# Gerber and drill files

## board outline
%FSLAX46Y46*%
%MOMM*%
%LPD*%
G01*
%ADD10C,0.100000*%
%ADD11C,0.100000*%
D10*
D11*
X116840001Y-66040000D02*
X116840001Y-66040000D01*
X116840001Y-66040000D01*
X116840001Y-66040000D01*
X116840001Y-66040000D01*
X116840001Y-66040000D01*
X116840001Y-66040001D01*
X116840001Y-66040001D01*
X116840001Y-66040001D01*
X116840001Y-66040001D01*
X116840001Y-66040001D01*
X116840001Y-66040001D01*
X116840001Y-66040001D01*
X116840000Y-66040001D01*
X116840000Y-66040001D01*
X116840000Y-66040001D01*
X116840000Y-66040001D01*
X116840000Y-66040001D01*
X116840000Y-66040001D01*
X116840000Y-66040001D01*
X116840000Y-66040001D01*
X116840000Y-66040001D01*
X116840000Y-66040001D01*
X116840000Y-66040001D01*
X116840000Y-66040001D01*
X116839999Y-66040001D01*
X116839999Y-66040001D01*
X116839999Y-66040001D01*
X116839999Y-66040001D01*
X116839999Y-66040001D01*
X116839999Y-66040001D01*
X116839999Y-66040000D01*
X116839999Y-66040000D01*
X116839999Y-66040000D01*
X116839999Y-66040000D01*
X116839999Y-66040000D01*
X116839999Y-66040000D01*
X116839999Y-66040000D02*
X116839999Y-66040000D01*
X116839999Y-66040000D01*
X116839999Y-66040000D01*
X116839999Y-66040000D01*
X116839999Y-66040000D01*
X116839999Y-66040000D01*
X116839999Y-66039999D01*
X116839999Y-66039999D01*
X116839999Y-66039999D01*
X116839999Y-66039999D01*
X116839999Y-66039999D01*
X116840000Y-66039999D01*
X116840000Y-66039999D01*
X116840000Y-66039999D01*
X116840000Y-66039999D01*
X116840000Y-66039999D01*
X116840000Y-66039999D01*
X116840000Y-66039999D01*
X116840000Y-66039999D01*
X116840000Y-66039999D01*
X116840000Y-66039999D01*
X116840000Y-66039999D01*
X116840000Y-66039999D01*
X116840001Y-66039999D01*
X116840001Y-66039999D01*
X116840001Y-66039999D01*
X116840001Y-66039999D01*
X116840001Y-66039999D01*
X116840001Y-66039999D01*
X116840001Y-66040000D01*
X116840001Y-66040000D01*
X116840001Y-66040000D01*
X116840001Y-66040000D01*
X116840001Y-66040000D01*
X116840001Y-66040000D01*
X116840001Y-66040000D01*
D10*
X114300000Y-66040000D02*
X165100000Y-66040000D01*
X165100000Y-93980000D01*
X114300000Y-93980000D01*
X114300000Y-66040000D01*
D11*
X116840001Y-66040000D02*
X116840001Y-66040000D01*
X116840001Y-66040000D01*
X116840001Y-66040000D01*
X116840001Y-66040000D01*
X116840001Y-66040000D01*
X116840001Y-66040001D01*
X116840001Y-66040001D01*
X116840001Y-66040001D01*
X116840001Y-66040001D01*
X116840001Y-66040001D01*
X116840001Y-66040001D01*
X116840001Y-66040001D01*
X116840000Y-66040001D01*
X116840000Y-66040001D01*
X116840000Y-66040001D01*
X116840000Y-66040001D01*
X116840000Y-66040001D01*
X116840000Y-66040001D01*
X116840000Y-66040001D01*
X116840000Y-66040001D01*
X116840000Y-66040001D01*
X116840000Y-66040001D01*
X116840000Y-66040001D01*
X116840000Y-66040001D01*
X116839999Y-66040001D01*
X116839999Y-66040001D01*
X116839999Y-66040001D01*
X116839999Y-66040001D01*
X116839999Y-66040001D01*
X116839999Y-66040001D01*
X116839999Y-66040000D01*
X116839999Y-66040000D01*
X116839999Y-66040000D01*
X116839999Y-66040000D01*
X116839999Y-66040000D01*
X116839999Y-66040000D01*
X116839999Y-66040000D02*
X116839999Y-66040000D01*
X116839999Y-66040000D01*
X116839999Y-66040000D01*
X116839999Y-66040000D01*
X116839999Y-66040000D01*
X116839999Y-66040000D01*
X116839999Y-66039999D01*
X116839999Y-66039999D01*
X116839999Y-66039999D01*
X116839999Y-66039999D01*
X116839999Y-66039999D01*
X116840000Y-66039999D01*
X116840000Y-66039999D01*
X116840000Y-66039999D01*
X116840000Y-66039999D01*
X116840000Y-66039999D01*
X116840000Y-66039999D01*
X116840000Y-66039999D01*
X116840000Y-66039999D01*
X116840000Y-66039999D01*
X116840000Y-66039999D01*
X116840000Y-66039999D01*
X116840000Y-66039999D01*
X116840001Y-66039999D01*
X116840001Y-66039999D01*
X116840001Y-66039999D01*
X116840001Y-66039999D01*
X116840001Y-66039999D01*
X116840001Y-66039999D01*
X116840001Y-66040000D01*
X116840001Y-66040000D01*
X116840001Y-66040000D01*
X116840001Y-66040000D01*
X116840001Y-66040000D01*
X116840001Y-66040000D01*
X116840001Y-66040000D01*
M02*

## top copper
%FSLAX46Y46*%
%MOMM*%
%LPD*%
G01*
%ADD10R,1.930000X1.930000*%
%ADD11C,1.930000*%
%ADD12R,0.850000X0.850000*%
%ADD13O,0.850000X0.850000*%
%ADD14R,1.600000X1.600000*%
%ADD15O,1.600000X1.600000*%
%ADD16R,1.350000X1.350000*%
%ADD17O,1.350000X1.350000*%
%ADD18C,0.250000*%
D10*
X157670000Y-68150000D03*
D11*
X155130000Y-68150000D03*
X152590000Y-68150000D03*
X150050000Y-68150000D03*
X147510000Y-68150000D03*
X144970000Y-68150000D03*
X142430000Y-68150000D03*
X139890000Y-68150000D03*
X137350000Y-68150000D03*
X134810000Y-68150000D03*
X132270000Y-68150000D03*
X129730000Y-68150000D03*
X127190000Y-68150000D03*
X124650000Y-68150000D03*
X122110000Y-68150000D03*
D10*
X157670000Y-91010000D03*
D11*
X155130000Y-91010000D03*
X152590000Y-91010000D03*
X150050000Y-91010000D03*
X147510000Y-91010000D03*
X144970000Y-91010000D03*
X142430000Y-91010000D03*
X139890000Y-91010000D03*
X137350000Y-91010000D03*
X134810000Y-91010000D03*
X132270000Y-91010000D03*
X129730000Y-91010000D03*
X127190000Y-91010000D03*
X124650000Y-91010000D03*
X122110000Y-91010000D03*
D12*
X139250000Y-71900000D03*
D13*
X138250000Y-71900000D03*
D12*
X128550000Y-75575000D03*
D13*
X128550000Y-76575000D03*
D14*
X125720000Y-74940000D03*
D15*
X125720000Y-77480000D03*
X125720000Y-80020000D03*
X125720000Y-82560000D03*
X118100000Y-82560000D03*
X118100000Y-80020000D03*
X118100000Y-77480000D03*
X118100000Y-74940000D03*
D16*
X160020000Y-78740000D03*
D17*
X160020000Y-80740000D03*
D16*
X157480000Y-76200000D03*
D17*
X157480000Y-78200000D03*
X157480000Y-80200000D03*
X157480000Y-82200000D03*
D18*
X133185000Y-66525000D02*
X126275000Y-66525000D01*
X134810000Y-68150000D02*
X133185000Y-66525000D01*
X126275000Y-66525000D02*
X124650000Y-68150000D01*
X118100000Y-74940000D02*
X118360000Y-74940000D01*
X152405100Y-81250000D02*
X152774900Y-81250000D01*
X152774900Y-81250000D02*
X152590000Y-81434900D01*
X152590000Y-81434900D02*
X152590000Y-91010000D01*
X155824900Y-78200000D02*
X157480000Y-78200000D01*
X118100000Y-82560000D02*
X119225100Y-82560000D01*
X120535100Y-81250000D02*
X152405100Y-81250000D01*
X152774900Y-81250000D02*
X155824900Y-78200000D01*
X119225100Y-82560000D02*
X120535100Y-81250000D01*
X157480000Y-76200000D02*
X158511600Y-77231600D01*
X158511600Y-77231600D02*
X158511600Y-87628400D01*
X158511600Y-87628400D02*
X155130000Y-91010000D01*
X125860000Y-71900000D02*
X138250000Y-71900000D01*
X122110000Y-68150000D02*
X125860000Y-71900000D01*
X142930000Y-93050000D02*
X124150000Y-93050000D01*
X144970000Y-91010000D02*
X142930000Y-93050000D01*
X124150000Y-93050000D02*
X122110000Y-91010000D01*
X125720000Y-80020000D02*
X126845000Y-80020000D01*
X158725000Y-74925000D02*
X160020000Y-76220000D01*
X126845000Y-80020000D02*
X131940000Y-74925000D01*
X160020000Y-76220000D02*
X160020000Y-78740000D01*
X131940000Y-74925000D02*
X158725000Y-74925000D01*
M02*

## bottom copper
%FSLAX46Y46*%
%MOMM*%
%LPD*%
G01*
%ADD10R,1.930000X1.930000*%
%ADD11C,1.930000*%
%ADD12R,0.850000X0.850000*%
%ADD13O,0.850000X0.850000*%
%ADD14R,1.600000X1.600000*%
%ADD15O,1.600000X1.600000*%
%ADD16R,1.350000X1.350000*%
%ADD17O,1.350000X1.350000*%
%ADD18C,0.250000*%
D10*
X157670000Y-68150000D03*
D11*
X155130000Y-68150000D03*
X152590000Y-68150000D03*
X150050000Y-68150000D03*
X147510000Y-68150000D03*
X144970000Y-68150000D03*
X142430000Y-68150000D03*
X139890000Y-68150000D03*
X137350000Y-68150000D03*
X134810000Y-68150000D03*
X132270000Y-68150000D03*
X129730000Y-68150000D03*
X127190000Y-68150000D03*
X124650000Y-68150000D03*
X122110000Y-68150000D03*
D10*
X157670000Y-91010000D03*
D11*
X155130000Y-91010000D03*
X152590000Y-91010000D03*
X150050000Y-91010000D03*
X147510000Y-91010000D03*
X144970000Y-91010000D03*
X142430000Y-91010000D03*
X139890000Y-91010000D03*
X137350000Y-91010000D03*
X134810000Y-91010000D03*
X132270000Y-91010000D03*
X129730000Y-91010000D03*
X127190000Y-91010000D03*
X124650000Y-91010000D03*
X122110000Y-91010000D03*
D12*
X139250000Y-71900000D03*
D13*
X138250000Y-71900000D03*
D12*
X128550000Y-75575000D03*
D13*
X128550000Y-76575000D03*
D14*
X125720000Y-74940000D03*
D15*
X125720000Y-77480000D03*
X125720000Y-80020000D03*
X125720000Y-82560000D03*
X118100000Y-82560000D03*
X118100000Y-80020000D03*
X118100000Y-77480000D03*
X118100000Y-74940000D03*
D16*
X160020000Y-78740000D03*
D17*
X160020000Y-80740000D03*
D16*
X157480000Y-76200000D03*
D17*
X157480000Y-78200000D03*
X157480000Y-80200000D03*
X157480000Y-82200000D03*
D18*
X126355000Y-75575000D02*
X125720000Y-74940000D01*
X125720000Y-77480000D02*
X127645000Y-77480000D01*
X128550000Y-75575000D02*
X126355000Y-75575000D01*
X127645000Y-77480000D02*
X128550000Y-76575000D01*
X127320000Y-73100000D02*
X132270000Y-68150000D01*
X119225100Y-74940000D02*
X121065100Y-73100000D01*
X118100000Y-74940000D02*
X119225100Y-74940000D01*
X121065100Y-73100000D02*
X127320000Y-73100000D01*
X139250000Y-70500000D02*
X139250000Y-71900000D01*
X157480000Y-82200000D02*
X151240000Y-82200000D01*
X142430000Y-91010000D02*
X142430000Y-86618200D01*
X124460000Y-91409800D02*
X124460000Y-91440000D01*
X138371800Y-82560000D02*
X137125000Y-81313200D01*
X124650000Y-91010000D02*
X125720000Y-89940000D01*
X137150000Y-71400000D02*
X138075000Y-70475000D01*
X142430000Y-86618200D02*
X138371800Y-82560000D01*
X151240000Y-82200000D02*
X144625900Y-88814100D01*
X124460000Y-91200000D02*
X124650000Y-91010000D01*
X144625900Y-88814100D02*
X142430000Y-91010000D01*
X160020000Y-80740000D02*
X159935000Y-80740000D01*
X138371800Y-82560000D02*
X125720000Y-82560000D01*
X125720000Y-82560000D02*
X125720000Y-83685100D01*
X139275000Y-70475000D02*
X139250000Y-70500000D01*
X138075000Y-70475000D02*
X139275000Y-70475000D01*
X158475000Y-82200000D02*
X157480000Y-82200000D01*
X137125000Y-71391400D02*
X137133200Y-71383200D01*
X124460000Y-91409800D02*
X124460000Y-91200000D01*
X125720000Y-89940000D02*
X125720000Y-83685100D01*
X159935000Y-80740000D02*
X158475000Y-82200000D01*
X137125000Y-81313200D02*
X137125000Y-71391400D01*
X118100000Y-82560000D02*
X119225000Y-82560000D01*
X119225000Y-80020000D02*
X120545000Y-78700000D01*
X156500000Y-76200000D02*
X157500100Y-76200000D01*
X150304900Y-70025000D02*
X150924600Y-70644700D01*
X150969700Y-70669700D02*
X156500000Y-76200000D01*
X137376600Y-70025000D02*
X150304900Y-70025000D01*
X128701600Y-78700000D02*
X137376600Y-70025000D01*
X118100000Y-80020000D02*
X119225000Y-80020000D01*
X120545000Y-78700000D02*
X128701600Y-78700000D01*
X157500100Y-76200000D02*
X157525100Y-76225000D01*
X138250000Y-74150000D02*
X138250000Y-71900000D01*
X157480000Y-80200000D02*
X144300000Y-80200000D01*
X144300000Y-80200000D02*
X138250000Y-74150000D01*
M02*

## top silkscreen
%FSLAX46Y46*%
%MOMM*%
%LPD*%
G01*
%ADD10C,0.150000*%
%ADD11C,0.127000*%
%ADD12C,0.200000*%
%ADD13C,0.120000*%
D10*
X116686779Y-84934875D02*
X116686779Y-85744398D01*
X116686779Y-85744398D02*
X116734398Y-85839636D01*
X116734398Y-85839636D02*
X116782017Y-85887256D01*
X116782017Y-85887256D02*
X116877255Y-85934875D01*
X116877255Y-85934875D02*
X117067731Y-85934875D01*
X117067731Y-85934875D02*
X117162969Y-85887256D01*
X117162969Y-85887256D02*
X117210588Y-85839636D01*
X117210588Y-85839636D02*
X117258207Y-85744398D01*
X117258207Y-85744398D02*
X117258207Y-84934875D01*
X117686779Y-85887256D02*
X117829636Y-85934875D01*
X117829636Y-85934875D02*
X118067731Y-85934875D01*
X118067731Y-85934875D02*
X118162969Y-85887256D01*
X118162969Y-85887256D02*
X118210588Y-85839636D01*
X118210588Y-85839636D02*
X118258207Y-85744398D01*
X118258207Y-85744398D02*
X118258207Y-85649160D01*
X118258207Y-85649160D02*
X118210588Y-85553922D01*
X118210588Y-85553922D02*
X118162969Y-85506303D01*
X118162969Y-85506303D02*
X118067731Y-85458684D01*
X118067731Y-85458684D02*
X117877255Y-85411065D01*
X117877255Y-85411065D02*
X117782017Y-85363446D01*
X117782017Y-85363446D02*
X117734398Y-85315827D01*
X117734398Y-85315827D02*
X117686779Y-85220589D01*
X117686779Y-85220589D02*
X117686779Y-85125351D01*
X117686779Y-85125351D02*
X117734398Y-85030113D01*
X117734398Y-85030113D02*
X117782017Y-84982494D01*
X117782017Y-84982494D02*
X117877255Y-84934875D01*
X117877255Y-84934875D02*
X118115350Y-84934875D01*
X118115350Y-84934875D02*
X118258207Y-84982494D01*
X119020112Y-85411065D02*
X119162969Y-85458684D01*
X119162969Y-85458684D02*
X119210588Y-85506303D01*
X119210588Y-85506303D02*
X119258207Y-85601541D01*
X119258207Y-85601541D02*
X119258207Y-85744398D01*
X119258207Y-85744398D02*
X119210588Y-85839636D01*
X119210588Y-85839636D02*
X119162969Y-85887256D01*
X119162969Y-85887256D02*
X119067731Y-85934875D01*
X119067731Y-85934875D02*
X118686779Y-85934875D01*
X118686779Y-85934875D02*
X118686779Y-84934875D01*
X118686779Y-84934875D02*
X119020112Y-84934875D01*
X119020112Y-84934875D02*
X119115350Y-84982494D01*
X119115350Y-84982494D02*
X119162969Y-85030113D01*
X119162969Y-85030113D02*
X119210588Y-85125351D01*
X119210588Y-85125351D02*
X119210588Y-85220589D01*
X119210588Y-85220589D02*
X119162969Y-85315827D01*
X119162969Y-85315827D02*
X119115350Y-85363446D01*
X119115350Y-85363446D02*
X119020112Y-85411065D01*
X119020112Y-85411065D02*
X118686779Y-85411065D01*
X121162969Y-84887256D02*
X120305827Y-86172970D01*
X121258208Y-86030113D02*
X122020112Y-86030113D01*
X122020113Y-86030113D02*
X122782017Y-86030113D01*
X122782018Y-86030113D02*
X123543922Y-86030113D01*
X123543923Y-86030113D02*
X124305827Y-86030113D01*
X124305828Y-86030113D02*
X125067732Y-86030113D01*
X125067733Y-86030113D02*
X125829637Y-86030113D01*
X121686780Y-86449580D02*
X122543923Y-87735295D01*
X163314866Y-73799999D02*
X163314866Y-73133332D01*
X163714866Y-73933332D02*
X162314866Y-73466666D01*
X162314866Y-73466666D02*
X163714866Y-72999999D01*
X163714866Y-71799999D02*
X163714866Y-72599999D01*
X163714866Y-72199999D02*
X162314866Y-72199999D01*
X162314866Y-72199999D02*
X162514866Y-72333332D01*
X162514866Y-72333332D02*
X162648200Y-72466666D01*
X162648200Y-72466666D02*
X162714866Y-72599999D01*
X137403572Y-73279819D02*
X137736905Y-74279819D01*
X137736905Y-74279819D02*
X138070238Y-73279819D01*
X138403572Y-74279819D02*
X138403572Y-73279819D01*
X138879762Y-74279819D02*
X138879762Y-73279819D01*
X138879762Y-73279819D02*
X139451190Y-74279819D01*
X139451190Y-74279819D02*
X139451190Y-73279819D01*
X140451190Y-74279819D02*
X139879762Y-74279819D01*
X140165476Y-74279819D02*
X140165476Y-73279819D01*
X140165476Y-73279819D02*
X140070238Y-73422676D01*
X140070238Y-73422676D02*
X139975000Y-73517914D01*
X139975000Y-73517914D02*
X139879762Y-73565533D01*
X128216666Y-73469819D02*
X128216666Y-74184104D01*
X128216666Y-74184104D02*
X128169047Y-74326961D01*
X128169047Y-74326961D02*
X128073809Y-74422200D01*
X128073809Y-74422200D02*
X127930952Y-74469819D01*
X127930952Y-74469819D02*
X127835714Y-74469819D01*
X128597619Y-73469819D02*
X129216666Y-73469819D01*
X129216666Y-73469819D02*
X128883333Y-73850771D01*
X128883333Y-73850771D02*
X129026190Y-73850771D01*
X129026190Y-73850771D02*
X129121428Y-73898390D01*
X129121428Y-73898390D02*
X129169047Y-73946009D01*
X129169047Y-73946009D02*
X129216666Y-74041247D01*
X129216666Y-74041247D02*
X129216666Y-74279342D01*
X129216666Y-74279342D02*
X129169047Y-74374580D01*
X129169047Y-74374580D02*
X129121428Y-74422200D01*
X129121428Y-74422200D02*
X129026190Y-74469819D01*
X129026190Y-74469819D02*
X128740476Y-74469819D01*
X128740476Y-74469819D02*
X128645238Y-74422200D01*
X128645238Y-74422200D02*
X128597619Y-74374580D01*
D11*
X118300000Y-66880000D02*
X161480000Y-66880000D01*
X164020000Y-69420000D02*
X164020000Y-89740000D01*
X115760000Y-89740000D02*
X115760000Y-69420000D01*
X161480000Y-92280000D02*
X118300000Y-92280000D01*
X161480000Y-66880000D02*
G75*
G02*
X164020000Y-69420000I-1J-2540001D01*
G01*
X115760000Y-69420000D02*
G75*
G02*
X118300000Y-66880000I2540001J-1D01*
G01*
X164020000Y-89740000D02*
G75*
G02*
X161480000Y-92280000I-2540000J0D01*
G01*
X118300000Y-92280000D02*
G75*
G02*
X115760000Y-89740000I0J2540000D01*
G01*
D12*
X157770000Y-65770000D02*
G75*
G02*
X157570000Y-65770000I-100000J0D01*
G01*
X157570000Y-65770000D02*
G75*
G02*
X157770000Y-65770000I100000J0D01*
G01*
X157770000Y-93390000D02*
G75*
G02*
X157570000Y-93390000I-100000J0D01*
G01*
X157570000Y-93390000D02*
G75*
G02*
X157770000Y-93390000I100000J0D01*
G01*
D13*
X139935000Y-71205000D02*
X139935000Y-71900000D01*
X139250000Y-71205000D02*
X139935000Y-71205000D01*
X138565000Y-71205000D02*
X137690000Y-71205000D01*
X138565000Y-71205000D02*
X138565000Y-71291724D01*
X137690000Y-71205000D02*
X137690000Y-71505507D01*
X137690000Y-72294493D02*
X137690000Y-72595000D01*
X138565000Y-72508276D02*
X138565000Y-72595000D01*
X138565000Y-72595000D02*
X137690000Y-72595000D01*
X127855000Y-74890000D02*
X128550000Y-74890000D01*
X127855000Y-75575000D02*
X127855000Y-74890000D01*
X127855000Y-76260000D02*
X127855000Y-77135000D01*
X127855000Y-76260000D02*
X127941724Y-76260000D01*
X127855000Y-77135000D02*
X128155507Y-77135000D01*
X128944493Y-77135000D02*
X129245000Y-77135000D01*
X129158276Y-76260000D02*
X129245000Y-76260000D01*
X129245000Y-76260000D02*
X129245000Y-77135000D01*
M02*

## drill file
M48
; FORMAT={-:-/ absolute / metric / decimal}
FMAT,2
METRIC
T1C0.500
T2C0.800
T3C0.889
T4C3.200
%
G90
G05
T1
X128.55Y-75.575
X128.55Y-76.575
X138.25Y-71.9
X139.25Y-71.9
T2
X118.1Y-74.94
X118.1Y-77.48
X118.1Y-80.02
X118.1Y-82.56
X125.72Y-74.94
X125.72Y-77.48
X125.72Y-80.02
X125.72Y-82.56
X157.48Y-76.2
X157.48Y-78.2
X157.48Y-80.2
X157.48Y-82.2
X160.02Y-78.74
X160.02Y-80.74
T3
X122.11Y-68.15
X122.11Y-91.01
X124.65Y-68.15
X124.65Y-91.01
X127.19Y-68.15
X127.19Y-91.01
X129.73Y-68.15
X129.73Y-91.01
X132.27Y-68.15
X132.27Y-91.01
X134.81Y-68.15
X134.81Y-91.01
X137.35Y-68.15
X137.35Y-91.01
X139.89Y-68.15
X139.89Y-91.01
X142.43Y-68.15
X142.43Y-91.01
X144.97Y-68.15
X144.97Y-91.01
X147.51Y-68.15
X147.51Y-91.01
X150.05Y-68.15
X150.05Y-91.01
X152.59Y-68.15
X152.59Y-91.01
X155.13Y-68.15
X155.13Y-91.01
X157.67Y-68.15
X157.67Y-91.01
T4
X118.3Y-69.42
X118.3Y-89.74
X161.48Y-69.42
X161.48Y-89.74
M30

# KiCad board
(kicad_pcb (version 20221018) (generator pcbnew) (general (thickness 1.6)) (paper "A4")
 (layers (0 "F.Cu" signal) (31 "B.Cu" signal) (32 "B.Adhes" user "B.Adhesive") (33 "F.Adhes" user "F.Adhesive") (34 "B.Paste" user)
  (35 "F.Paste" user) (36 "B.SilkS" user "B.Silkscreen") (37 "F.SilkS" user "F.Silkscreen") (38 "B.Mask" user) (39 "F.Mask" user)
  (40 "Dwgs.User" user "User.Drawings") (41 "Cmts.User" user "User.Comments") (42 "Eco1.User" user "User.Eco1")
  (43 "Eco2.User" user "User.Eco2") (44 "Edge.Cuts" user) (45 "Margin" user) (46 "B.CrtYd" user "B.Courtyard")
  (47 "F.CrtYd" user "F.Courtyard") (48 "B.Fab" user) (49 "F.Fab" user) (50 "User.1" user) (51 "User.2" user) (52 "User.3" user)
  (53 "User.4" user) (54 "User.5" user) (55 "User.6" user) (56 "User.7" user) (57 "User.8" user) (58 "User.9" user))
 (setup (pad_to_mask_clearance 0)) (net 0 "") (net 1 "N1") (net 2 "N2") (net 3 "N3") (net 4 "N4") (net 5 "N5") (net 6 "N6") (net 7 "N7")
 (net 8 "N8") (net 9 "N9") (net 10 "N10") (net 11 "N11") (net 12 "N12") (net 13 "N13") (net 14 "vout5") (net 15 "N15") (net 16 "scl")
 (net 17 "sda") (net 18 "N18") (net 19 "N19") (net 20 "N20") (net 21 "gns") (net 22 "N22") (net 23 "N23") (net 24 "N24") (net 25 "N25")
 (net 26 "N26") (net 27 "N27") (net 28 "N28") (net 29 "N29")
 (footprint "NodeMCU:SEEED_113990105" (layer "F.Cu") (at 139.89 79.58 -90)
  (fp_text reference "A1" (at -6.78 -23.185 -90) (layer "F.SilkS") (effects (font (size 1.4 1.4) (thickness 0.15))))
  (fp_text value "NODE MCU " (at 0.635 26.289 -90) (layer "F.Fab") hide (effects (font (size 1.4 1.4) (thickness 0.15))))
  (fp_line (start -12.7 21.59) (end -12.7 -21.59) (stroke (width 0.127) (type solid)) (layer "F.SilkS"))
  (fp_line (start -10.16 -24.13) (end 10.16 -24.13) (stroke (width 0.127) (type solid)) (layer "F.SilkS"))
  (fp_line (start 10.16 24.13) (end -10.16 24.13) (stroke (width 0.127) (type solid)) (layer "F.SilkS"))
  (fp_line (start 12.7 -21.59) (end 12.7 21.59) (stroke (width 0.127) (type solid)) (layer "F.SilkS"))
  (fp_arc (start -12.7 -21.59) (mid -11.956051 -23.386051) (end -10.16 -24.13) (stroke (width 0.127) (type solid)) (layer "F.SilkS"))
  (fp_arc (start -10.16 24.13) (mid -11.956051 23.386051) (end -12.7 21.59) (stroke (width 0.127) (type solid)) (layer "F.SilkS"))
  (fp_arc (start 10.16 -24.13) (mid 11.956051 -23.386051) (end 12.7 -21.59) (stroke (width 0.127) (type solid)) (layer "F.SilkS"))
  (fp_arc (start 12.7 21.59) (mid 11.956051 23.386051) (end 10.16 24.13) (stroke (width 0.127) (type solid)) (layer "F.SilkS"))
  (fp_circle (center -13.81 -17.78) (end -13.71 -17.78) (stroke (width 0.2) (type solid)) (fill none) (layer "F.SilkS"))
  (fp_circle (center 13.81 -17.78) (end 13.91 -17.78) (stroke (width 0.2) (type solid)) (fill none) (layer "F.SilkS"))
  (pad "" np_thru_hole circle (at -10.16 -21.59 270) (size 3.2 3.2) (drill 3.2) (layers "*.Cu" "*.Mask"))
  (pad "" np_thru_hole circle (at -10.16 21.59 270) (size 3.2 3.2) (drill 3.2) (layers "*.Cu" "*.Mask"))
  (pad "" np_thru_hole circle (at 10.16 -21.59 270) (size 3.2 3.2) (drill 3.2) (layers "*.Cu" "*.Mask"))
  (pad "" np_thru_hole circle (at 10.16 21.59 270) (size 3.2 3.2) (drill 3.2) (layers "*.Cu" "*.Mask"))
  (pad "J1_1" thru_hole rect (at -11.43 -17.78 270) (size 1.93 1.93) (drill 0.889) (layers "*.Cu" "*.Mask") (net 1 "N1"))
  (pad "J1_2" thru_hole circle (at -11.43 -15.24 270) (size 1.93 1.93) (drill 0.889) (layers "*.Cu" "*.Mask") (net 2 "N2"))
  (pad "J1_3" thru_hole circle (at -11.43 -12.7 270) (size 1.93 1.93) (drill 0.889) (layers "*.Cu" "*.Mask") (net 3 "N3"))
  (pad "J1_4" thru_hole circle (at -11.43 -10.16 270) (size 1.93 1.93) (drill 0.889) (layers "*.Cu" "*.Mask") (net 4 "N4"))
  (pad "J1_5" thru_hole circle (at -11.43 -7.62 270) (size 1.93 1.93) (drill 0.889) (layers "*.Cu" "*.Mask") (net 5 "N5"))
  (pad "J1_6" thru_hole circle (at -11.43 -5.08 270) (size 1.93 1.93) (drill 0.889) (layers "*.Cu" "*.Mask") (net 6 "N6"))
  (pad "J1_7" thru_hole circle (at -11.43 -2.54 270) (size 1.93 1.93) (drill 0.889) (layers "*.Cu" "*.Mask") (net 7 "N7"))
  (pad "J1_8" thru_hole circle (at -11.43 0 270) (size 1.93 1.93) (drill 0.889) (layers "*.Cu" "*.Mask") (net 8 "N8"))
  (pad "J1_9" thru_hole circle (at -11.43 2.54 270) (size 1.93 1.93) (drill 0.889) (layers "*.Cu" "*.Mask") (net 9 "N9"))
  (pad "J1_10" thru_hole circle (at -11.43 5.08 270) (size 1.93 1.93) (drill 0.889) (layers "*.Cu" "*.Mask") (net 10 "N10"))
  (pad "J1_11" thru_hole circle (at -11.43 7.62 270) (size 1.93 1.93) (drill 0.889) (layers "*.Cu" "*.Mask") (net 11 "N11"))
  (pad "J1_12" thru_hole circle (at -11.43 10.16 270) (size 1.93 1.93) (drill 0.889) (layers "*.Cu" "*.Mask") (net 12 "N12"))
  (pad "J1_13" thru_hole circle (at -11.43 12.7 270) (size 1.93 1.93) (drill 0.889) (layers "*.Cu" "*.Mask") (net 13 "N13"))
  (pad "J1_14" thru_hole circle (at -11.43 15.24 270) (size 1.93 1.93) (drill 0.889) (layers "*.Cu" "*.Mask") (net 10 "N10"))
  (pad "J1_15" thru_hole circle (at -11.43 17.78 270) (size 1.93 1.93) (drill 0.889) (layers "*.Cu" "*.Mask") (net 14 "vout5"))
  (pad "J2_1" thru_hole rect (at 11.43 -17.78 270) (size 1.93 1.93) (drill 0.889) (layers "*.Cu" "*.Mask") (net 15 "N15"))
  (pad "J2_2" thru_hole circle (at 11.43 -15.24 270) (size 1.93 1.93) (drill 0.889) (layers "*.Cu" "*.Mask") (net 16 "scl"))
  (pad "J2_3" thru_hole circle (at 11.43 -12.7 270) (size 1.93 1.93) (drill 0.889) (layers "*.Cu" "*.Mask") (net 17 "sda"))
  (pad "J2_4" thru_hole circle (at 11.43 -10.16 270) (size 1.93 1.93) (drill 0.889) (layers "*.Cu" "*.Mask") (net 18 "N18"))
  (pad "J2_5" thru_hole circle (at 11.43 -7.62 270) (size 1.93 1.93) (drill 0.889) (layers "*.Cu" "*.Mask") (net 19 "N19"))
  (pad "J2_6" thru_hole circle (at 11.43 -5.08 270) (size 1.93 1.93) (drill 0.889) (layers "*.Cu" "*.Mask") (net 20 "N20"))
  (pad "J2_7" thru_hole circle (at 11.43 -2.54 270) (size 1.93 1.93) (drill 0.889) (layers "*.Cu" "*.Mask") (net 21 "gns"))
  (pad "J2_8" thru_hole circle (at 11.43 0 270) (size 1.93 1.93) (drill 0.889) (layers "*.Cu" "*.Mask") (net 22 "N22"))
  (pad "J2_9" thru_hole circle (at 11.43 2.54 270) (size 1.93 1.93) (drill 0.889) (layers "*.Cu" "*.Mask") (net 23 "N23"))
  (pad "J2_10" thru_hole circle (at 11.43 5.08 270) (size 1.93 1.93) (drill 0.889) (layers "*.Cu" "*.Mask") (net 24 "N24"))
  (pad "J2_11" thru_hole circle (at 11.43 7.62 270) (size 1.93 1.93) (drill 0.889) (layers "*.Cu" "*.Mask") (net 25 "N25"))
  (pad "J2_12" thru_hole circle (at 11.43 10.16 270) (size 1.93 1.93) (drill 0.889) (layers "*.Cu" "*.Mask") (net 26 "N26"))
  (pad "J2_13" thru_hole circle (at 11.43 12.7 270) (size 1.93 1.93) (drill 0.889) (layers "*.Cu" "*.Mask") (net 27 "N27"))
  (pad "J2_14" thru_hole circle (at 11.43 15.24 270) (size 1.93 1.93) (drill 0.889) (layers "*.Cu" "*.Mask") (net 21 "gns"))
  (pad "J2_15" thru_hole circle (at 11.43 17.78 270) (size 1.93 1.93) (drill 0.889) (layers "*.Cu" "*.Mask") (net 20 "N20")))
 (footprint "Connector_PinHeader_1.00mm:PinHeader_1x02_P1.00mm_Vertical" (layer "F.Cu") (at 139.25 71.9 -90)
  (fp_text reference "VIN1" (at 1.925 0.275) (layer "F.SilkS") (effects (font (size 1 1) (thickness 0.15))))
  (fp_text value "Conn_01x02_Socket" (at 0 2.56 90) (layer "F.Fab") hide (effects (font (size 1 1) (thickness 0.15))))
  (fp_line (start -0.695 -0.685) (end 0 -0.685) (stroke (width 0.12) (type solid)) (layer "F.SilkS"))
  (fp_line (start -0.695 0) (end -0.695 -0.685) (stroke (width 0.12) (type solid)) (layer "F.SilkS"))
  (fp_line (start -0.695 0.685) (end -0.695 1.56) (stroke (width 0.12) (type solid)) (layer "F.SilkS"))
  (fp_line (start -0.695 0.685) (end -0.608276 0.685) (stroke (width 0.12) (type solid)) (layer "F.SilkS"))
  (fp_line (start -0.695 1.56) (end -0.394493 1.56) (stroke (width 0.12) (type solid)) (layer "F.SilkS"))
  (fp_line (start 0.394493 1.56) (end 0.695 1.56) (stroke (width 0.12) (type solid)) (layer "F.SilkS"))
  (fp_line (start 0.608276 0.685) (end 0.695 0.685) (stroke (width 0.12) (type solid)) (layer "F.SilkS"))
  (fp_line (start 0.695 0.685) (end 0.695 1.56) (stroke (width 0.12) (type solid)) (layer "F.SilkS"))
  (pad "1" thru_hole rect (at 0 0 270) (size 0.85 0.85) (drill 0.5) (layers "*.Cu" "*.Mask") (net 21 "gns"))
  (pad "2" thru_hole oval (at 0 1 270) (size 0.85 0.85) (drill 0.5) (layers "*.Cu" "*.Mask") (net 14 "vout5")))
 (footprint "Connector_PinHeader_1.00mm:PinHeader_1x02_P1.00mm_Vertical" (layer "F.Cu") (at 128.55 75.575)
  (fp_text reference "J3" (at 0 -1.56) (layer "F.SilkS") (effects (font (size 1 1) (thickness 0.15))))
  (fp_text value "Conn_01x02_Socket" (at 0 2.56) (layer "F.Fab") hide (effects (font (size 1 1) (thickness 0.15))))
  (fp_line (start -0.695 -0.685) (end 0 -0.685) (stroke (width 0.12) (type solid)) (layer "F.SilkS"))
  (fp_line (start -0.695 0) (end -0.695 -0.685) (stroke (width 0.12) (type solid)) (layer "F.SilkS"))
  (fp_line (start -0.695 0.685) (end -0.695 1.56) (stroke (width 0.12) (type solid)) (layer "F.SilkS"))
  (fp_line (start -0.695 0.685) (end -0.608276 0.685) (stroke (width 0.12) (type solid)) (layer "F.SilkS"))
  (fp_line (start -0.695 1.56) (end -0.394493 1.56) (stroke (width 0.12) (type solid)) (layer "F.SilkS"))
  (fp_line (start 0.394493 1.56) (end 0.695 1.56) (stroke (width 0.12) (type solid)) (layer "F.SilkS"))
  (fp_line (start 0.608276 0.685) (end 0.695 0.685) (stroke (width 0.12) (type solid)) (layer "F.SilkS"))
  (fp_line (start 0.695 0.685) (end 0.695 1.56) (stroke (width 0.12) (type solid)) (layer "F.SilkS"))
  (pad "1" thru_hole rect (at 0 0) (size 0.85 0.85) (drill 0.5) (layers "*.Cu" "*.Mask"))
  (pad "2" thru_hole oval (at 0 1) (size 0.85 0.85) (drill 0.5) (layers "*.Cu" "*.Mask")))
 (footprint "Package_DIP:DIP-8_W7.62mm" (layer "B.Cu") (at 125.72 74.94 180)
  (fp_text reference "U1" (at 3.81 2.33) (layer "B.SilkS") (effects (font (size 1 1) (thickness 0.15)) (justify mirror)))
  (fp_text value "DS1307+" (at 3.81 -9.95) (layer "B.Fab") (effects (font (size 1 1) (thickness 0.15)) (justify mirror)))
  (pad "1" thru_hole rect (at 0 0 180) (size 1.6 1.6) (drill 0.8) (layers "*.Cu" "*.Mask"))
  (pad "2" thru_hole oval (at 0 -2.54 180) (size 1.6 1.6) (drill 0.8) (layers "*.Cu" "*.Mask"))
  (pad "3" thru_hole oval (at 0 -5.08 180) (size 1.6 1.6) (drill 0.8) (layers "*.Cu" "*.Mask") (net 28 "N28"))
  (pad "4" thru_hole oval (at 0 -7.62 180) (size 1.6 1.6) (drill 0.8) (layers "*.Cu" "*.Mask") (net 21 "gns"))
  (pad "5" thru_hole oval (at 7.62 -7.62 180) (size 1.6 1.6) (drill 0.8) (layers "*.Cu" "*.Mask") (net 17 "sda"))
  (pad "6" thru_hole oval (at 7.62 -5.08 180) (size 1.6 1.6) (drill 0.8) (layers "*.Cu" "*.Mask") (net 16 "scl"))
  (pad "7" thru_hole oval (at 7.62 -2.54 180) (size 1.6 1.6) (drill 0.8) (layers "*.Cu" "*.Mask") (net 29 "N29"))
  (pad "8" thru_hole oval (at 7.62 0 180) (size 1.6 1.6) (drill 0.8) (layers "*.Cu" "*.Mask") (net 11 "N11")))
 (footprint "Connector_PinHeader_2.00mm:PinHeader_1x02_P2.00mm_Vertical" (layer "B.Cu") (at 160.02 78.74 180)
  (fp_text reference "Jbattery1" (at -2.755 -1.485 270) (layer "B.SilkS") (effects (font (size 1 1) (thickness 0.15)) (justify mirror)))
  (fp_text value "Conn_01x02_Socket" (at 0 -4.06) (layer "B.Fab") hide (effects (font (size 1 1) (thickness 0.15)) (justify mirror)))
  (pad "1" thru_hole rect (at 0 0 180) (size 1.35 1.35) (drill 0.8) (layers "*.Cu" "*.Mask") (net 28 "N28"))
  (pad "2" thru_hole oval (at 0 -2 180) (size 1.35 1.35) (drill 0.8) (layers "*.Cu" "*.Mask") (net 21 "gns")))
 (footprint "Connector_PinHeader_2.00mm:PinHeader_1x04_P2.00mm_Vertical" (layer "B.Cu") (at 157.48 76.2 180)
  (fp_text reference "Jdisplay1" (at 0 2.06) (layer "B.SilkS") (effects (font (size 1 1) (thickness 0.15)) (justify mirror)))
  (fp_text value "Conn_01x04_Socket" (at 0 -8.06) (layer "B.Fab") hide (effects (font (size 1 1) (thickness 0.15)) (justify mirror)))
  (pad "1" thru_hole rect (at 0 0 180) (size 1.35 1.35) (drill 0.8) (layers "*.Cu" "*.Mask") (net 16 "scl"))
  (pad "2" thru_hole oval (at 0 -2 180) (size 1.35 1.35) (drill 0.8) (layers "*.Cu" "*.Mask") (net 17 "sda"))
  (pad "3" thru_hole oval (at 0 -4 180) (size 1.35 1.35) (drill 0.8) (layers "*.Cu" "*.Mask") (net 14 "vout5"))
  (pad "4" thru_hole oval (at 0 -6 180) (size 1.35 1.35) (drill 0.8) (layers "*.Cu" "*.Mask") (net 21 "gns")))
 (gr_circle (center 116.84 66.04) (end 116.84 66.04) (stroke (width 0.1) (type default)) (fill none) (layer "Edge.Cuts"))
 (gr_rect (start 114.3 66.04) (end 165.1 93.98) (stroke (width 0.1) (type default)) (fill none) (layer "Edge.Cuts"))
 (gr_circle (center 116.84 66.04) (end 116.84 66.04) (stroke (width 0.1) (type default)) (fill none) (layer "Edge.Cuts"))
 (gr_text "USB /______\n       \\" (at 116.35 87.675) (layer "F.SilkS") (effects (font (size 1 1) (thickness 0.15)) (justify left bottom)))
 (segment (start 126.355 75.575) (end 125.72 74.94) (width 0.25) (layer "B.Cu") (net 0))
 (segment (start 125.72 77.48) (end 127.645 77.48) (width 0.25) (layer "B.Cu") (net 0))
 (segment (start 128.55 75.575) (end 126.355 75.575) (width 0.25) (layer "B.Cu") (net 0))
 (segment (start 127.645 77.48) (end 128.55 76.575) (width 0.25) (layer "B.Cu") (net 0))
 (segment (start 133.185 66.525) (end 126.275 66.525) (width 0.25) (layer "F.Cu") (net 10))
 (segment (start 134.81 68.15) (end 133.185 66.525) (width 0.25) (layer "F.Cu") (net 10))
 (segment (start 126.275 66.525) (end 124.65 68.15) (width 0.25) (layer "F.Cu") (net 10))
 (segment (start 118.1 74.94) (end 118.36 74.94) (width 0.25) (layer "F.Cu") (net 11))
 (segment (start 127.32 73.1) (end 132.27 68.15) (width 0.25) (layer "B.Cu") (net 11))
 (segment (start 119.2251 74.94) (end 121.0651 73.1) (width 0.25) (layer "B.Cu") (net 11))
 (segment (start 118.1 74.94) (end 119.2251 74.94) (width 0.25) (layer "B.Cu") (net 11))
 (segment (start 121.0651 73.1) (end 127.32 73.1) (width 0.25) (layer "B.Cu") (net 11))
 (segment (start 139.25 70.5) (end 139.25 71.9) (width 0.25) (layer "B.Cu") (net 21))
 (segment (start 157.48 82.2) (end 151.24 82.2) (width 0.25) (layer "B.Cu") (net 21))
 (segment (start 142.43 91.01) (end 142.43 86.6182) (width 0.25) (layer "B.Cu") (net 21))
 (segment (start 124.46 91.4098) (end 124.46 91.44) (width 0.25) (layer "B.Cu") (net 21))
 (segment (start 138.3718 82.56) (end 137.125 81.3132) (width 0.25) (layer "B.Cu") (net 21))
 (segment (start 124.65 91.01) (end 125.72 89.94) (width 0.25) (layer "B.Cu") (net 21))
 (segment (start 137.15 71.4) (end 138.075 70.475) (width 0.25) (layer "B.Cu") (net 21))
 (segment (start 142.43 86.6182) (end 138.3718 82.56) (width 0.25) (layer "B.Cu") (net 21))
 (segment (start 151.24 82.2) (end 144.6259 88.8141) (width 0.25) (layer "B.Cu") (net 21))
 (segment (start 124.46 91.2) (end 124.65 91.01) (width 0.25) (layer "B.Cu") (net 21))
 (segment (start 144.6259 88.8141) (end 142.43 91.01) (width 0.25) (layer "B.Cu") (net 21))
 (segment (start 160.02 80.74) (end 159.935 80.74) (width 0.25) (layer "B.Cu") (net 21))
 (segment (start 138.3718 82.56) (end 125.72 82.56) (width 0.25) (layer "B.Cu") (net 21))
 (segment (start 125.72 82.56) (end 125.72 83.6851) (width 0.25) (layer "B.Cu") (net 21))
 (segment (start 139.275 70.475) (end 139.25 70.5) (width 0.25) (layer "B.Cu") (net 21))
 (segment (start 138.075 70.475) (end 139.275 70.475) (width 0.25) (layer "B.Cu") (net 21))
 (segment (start 158.475 82.2) (end 157.48 82.2) (width 0.25) (layer "B.Cu") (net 21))
 (segment (start 137.125 71.3914) (end 137.1332 71.3832) (width 0.25) (layer "B.Cu") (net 21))
 (segment (start 124.46 91.4098) (end 124.46 91.2) (width 0.25) (layer "B.Cu") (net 21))
 (segment (start 125.72 89.94) (end 125.72 83.6851) (width 0.25) (layer "B.Cu") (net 21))
 (segment (start 159.935 80.74) (end 158.475 82.2) (width 0.25) (layer "B.Cu") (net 21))
 (segment (start 137.125 81.3132) (end 137.125 71.3914) (width 0.25) (layer "B.Cu") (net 21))
 (segment (start 152.4051 81.25) (end 152.7749 81.25) (width 0.25) (layer "F.Cu") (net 17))
 (segment (start 152.7749 81.25) (end 152.59 81.4349) (width 0.25) (layer "F.Cu") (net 17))
 (segment (start 152.59 81.4349) (end 152.59 91.01) (width 0.25) (layer "F.Cu") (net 17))
 (segment (start 155.8249 78.2) (end 157.48 78.2) (width 0.25) (layer "F.Cu") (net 17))
 (segment (start 118.1 82.56) (end 119.2251 82.56) (width 0.25) (layer "F.Cu") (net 17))
 (segment (start 120.5351 81.25) (end 152.4051 81.25) (width 0.25) (layer "F.Cu") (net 17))
 (segment (start 152.7749 81.25) (end 155.8249 78.2) (width 0.25) (layer "F.Cu") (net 17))
 (segment (start 119.2251 82.56) (end 120.5351 81.25) (width 0.25) (layer "F.Cu") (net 17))
 (segment (start 118.1 82.56) (end 119.225 82.56) (width 0.25) (layer "B.Cu") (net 17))
 (segment (start 157.48 76.2) (end 158.5116 77.2316) (width 0.25) (layer "F.Cu") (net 16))
 (segment (start 158.5116 77.2316) (end 158.5116 87.6284) (width 0.25) (layer "F.Cu") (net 16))
 (segment (start 158.5116 87.6284) (end 155.13 91.01) (width 0.25) (layer "F.Cu") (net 16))
 (segment (start 119.225 80.02) (end 120.545 78.7) (width 0.25) (layer "B.Cu") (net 16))
 (segment (start 156.5 76.2) (end 157.5001 76.2) (width 0.25) (layer "B.Cu") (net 16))
 (segment (start 150.3049 70.025) (end 150.9246 70.6447) (width 0.25) (layer "B.Cu") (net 16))
 (segment (start 150.9697 70.6697) (end 156.5 76.2) (width 0.25) (layer "B.Cu") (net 16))
 (segment (start 137.3766 70.025) (end 150.3049 70.025) (width 0.25) (layer "B.Cu") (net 16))
 (segment (start 128.7016 78.7) (end 137.3766 70.025) (width 0.25) (layer "B.Cu") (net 16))
 (segment (start 118.1 80.02) (end 119.225 80.02) (width 0.25) (layer "B.Cu") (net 16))
 (segment (start 120.545 78.7) (end 128.7016 78.7) (width 0.25) (layer "B.Cu") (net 16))
 (segment (start 157.5001 76.2) (end 157.5251 76.225) (width 0.25) (layer "B.Cu") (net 16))
 (segment (start 125.86 71.9) (end 138.25 71.9) (width 0.25) (layer "F.Cu") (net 14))
 (segment (start 122.11 68.15) (end 125.86 71.9) (width 0.25) (layer "F.Cu") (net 14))
 (segment (start 138.25 74.15) (end 138.25 71.9) (width 0.25) (layer "B.Cu") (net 14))
 (segment (start 157.48 80.2) (end 144.3 80.2) (width 0.25) (layer "B.Cu") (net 14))
 (segment (start 144.3 80.2) (end 138.25 74.15) (width 0.25) (layer "B.Cu") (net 14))
 (segment (start 142.93 93.05) (end 124.15 93.05) (width 0.25) (layer "F.Cu") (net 20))
 (segment (start 144.97 91.01) (end 142.93 93.05) (width 0.25) (layer "F.Cu") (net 20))
 (segment (start 124.15 93.05) (end 122.11 91.01) (width 0.25) (layer "F.Cu") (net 20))
 (segment (start 125.72 80.02) (end 126.845 80.02) (width 0.25) (layer "F.Cu") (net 28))
 (segment (start 158.725 74.925) (end 160.02 76.22) (width 0.25) (layer "F.Cu") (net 28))
 (segment (start 126.845 80.02) (end 131.94 74.925) (width 0.25) (layer "F.Cu") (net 28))
 (segment (start 160.02 76.22) (end 160.02 78.74) (width 0.25) (layer "F.Cu") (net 28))
 (segment (start 131.94 74.925) (end 158.725 74.925) (width 0.25) (layer "F.Cu") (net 28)))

